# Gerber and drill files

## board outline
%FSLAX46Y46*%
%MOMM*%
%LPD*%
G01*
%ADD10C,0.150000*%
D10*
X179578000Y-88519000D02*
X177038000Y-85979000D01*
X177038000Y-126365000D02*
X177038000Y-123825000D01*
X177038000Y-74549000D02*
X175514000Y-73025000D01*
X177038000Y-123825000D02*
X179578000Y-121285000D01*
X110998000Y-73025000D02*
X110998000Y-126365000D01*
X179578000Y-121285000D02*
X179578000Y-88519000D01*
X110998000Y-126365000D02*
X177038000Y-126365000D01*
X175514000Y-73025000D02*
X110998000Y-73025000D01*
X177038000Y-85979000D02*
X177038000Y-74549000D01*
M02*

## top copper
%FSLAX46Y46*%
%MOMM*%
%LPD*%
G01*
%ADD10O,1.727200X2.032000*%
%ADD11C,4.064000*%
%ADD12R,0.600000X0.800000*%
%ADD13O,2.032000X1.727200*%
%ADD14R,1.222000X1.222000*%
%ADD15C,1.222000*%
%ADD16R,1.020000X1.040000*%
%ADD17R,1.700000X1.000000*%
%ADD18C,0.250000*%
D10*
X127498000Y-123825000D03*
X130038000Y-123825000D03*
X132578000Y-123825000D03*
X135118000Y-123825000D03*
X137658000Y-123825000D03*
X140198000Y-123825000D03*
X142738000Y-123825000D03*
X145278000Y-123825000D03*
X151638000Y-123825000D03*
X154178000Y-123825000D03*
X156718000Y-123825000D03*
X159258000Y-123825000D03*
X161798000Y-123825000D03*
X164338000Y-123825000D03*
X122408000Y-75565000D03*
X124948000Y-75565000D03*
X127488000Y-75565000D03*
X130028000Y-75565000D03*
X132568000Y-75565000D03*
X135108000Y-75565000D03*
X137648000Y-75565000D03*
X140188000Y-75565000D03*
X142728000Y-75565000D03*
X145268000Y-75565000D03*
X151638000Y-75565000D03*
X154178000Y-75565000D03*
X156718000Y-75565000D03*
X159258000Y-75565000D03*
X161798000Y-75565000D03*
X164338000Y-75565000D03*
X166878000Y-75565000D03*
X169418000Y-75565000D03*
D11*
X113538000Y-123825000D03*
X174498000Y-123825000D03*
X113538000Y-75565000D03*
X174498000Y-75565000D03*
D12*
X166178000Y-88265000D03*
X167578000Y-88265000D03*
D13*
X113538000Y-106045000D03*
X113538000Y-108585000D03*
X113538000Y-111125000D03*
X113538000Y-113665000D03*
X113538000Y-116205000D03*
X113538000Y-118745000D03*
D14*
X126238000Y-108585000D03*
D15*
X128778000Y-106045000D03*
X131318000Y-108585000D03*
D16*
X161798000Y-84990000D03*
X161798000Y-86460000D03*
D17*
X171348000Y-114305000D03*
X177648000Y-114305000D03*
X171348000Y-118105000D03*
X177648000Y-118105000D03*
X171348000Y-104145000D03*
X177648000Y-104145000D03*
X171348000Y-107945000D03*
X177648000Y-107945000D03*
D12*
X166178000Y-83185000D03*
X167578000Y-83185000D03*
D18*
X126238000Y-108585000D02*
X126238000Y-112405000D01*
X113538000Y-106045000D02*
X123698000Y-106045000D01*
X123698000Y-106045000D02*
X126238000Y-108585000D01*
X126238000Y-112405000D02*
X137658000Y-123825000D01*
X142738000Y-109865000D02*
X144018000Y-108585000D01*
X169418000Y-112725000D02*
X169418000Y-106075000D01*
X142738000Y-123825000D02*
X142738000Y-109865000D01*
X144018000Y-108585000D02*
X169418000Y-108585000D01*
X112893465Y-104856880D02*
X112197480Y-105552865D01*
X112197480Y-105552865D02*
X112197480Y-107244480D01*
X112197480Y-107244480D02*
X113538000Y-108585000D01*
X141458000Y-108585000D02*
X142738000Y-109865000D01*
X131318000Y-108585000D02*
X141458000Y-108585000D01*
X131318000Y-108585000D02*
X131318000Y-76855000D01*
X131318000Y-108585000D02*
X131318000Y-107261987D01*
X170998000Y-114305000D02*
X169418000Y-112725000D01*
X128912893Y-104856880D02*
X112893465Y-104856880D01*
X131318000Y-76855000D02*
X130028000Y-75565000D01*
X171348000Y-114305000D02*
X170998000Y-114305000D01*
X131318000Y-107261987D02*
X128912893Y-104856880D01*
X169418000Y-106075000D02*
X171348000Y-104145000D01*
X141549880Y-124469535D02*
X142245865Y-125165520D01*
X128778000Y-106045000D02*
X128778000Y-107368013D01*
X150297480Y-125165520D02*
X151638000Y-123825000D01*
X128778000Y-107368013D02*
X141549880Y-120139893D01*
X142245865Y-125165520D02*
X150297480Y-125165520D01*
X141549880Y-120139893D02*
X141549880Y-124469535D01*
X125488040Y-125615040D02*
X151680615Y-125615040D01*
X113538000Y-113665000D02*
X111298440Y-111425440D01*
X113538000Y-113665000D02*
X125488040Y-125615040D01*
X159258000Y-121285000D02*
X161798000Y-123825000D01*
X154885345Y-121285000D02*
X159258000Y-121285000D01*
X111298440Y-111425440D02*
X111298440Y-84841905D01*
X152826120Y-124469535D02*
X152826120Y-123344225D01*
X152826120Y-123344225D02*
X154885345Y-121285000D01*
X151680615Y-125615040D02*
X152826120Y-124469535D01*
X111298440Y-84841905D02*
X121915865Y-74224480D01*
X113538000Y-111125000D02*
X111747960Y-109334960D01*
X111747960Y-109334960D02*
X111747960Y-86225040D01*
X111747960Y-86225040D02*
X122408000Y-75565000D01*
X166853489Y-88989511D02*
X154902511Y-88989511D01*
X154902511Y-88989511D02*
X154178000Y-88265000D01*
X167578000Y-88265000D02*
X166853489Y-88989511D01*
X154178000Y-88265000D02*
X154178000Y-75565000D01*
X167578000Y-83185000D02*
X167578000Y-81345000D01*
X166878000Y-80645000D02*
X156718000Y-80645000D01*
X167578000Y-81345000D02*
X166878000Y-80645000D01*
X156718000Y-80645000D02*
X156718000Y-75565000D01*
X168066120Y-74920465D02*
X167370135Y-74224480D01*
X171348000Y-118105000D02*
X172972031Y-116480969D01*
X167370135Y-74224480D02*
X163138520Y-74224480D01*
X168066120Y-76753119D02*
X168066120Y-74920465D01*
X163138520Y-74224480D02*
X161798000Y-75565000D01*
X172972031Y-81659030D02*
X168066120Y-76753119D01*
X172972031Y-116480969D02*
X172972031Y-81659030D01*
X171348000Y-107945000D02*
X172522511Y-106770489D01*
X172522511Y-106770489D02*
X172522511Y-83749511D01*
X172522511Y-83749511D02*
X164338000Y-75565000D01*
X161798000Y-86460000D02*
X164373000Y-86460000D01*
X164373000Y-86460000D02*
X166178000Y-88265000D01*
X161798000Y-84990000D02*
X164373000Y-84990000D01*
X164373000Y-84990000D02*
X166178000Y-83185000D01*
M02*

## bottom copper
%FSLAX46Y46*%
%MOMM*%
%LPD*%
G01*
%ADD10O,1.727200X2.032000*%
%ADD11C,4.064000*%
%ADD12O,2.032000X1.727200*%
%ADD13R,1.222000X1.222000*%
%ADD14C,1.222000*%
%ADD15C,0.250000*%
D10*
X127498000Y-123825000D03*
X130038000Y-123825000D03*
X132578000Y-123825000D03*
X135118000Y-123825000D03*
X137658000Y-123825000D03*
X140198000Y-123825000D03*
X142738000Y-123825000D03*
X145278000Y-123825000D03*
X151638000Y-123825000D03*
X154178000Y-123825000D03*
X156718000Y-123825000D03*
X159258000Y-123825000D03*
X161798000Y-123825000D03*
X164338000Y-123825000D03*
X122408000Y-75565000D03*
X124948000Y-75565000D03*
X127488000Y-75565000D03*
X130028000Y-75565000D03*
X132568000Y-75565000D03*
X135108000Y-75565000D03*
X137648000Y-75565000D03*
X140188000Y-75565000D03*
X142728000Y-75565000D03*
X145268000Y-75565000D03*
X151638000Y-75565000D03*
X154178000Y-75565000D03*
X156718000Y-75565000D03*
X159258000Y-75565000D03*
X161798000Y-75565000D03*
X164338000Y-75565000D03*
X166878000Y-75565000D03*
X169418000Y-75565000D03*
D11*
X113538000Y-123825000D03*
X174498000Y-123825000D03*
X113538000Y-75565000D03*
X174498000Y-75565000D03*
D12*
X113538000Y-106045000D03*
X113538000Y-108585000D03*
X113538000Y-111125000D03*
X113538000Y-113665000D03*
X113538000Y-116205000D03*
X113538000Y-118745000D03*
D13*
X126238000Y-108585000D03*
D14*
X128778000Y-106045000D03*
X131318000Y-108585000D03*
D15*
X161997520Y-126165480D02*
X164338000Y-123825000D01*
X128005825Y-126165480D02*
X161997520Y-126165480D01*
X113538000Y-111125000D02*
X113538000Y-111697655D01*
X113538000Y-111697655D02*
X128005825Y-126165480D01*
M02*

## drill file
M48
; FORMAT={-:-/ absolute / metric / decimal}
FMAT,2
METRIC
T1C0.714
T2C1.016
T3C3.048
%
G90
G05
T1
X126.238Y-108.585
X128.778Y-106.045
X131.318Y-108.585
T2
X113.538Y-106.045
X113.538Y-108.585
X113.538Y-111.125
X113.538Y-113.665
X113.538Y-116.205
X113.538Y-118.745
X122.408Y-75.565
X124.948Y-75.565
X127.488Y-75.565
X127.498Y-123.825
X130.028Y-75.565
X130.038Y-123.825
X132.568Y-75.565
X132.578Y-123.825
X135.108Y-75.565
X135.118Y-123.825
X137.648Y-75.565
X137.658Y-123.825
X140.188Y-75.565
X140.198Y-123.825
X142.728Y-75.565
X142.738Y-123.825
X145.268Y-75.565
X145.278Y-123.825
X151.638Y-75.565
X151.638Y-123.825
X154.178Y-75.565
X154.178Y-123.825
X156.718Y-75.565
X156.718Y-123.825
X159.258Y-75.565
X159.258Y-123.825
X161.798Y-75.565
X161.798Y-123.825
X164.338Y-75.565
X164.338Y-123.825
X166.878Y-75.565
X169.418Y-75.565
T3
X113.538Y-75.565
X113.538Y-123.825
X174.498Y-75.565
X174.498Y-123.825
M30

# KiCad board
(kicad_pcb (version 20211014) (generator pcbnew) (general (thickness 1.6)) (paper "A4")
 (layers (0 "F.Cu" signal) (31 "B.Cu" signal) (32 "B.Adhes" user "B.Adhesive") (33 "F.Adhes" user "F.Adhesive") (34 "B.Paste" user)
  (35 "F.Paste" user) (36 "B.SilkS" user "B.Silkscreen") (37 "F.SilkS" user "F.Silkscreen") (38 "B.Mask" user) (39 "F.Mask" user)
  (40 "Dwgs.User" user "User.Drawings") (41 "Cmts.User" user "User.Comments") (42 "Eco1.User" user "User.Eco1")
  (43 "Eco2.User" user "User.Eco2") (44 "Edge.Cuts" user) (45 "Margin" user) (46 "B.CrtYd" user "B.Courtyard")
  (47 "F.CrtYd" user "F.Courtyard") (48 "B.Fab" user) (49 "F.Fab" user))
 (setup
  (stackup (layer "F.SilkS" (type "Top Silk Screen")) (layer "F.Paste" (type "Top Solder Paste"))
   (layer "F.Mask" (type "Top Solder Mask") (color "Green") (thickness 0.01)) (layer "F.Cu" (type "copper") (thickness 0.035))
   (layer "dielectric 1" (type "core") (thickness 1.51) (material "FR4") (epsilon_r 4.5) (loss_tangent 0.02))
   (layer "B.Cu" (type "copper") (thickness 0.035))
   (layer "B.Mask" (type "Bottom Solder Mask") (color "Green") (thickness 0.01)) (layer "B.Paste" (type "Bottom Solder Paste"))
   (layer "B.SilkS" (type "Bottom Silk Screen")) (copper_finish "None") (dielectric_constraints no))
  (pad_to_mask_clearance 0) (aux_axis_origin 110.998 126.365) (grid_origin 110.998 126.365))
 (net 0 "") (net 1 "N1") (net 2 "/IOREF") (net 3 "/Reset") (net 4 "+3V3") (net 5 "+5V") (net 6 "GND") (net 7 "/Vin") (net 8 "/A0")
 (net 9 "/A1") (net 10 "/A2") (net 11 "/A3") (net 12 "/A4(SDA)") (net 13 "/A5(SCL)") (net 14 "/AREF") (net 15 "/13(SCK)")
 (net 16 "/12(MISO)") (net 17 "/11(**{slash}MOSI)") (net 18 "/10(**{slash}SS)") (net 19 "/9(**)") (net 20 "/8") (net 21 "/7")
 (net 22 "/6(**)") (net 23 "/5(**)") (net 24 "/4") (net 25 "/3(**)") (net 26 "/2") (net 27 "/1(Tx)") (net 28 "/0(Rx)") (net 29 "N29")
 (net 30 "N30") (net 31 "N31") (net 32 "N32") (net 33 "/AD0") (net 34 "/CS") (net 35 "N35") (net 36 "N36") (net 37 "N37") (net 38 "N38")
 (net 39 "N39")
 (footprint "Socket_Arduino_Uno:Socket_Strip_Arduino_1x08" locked (layer "F.Cu") (at 127.498 123.825)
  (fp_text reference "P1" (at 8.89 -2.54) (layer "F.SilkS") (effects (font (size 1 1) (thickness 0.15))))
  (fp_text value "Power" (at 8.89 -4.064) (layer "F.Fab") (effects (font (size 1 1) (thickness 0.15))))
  (pad "1" thru_hole oval locked (at 0 0) (size 1.7272 2.032) (drill 1.016) (layers *.Cu *.Mask "F.SilkS") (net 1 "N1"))
  (pad "2" thru_hole oval locked (at 2.54 0) (size 1.7272 2.032) (drill 1.016) (layers *.Cu *.Mask "F.SilkS") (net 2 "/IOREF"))
  (pad "3" thru_hole oval locked (at 5.08 0) (size 1.7272 2.032) (drill 1.016) (layers *.Cu *.Mask "F.SilkS") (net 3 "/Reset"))
  (pad "4" thru_hole oval locked (at 7.62 0) (size 1.7272 2.032) (drill 1.016) (layers *.Cu *.Mask "F.SilkS") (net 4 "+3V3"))
  (pad "5" thru_hole oval locked (at 10.16 0) (size 1.7272 2.032) (drill 1.016) (layers *.Cu *.Mask "F.SilkS") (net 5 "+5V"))
  (pad "6" thru_hole oval locked (at 12.7 0) (size 1.7272 2.032) (drill 1.016) (layers *.Cu *.Mask "F.SilkS") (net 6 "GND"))
  (pad "7" thru_hole oval locked (at 15.24 0) (size 1.7272 2.032) (drill 1.016) (layers *.Cu *.Mask "F.SilkS") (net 6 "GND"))
  (pad "8" thru_hole oval locked (at 17.78 0) (size 1.7272 2.032) (drill 1.016) (layers *.Cu *.Mask "F.SilkS") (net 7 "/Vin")))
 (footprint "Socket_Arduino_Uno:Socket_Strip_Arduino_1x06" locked (layer "F.Cu") (at 151.638 123.825)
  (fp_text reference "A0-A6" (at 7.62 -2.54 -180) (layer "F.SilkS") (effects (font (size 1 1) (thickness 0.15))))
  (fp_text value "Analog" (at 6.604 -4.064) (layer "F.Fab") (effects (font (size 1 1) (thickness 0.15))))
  (pad "1" thru_hole oval locked (at 0 0) (size 1.7272 2.032) (drill 1.016) (layers *.Cu *.Mask "F.SilkS") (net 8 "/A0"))
  (pad "2" thru_hole oval locked (at 2.54 0) (size 1.7272 2.032) (drill 1.016) (layers *.Cu *.Mask "F.SilkS") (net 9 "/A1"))
  (pad "3" thru_hole oval locked (at 5.08 0) (size 1.7272 2.032) (drill 1.016) (layers *.Cu *.Mask "F.SilkS") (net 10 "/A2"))
  (pad "4" thru_hole oval locked (at 7.62 0) (size 1.7272 2.032) (drill 1.016) (layers *.Cu *.Mask "F.SilkS") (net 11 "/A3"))
  (pad "5" thru_hole oval locked (at 10.16 0) (size 1.7272 2.032) (drill 1.016) (layers *.Cu *.Mask "F.SilkS") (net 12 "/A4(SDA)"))
  (pad "6" thru_hole oval locked (at 12.7 0) (size 1.7272 2.032) (drill 1.016) (layers *.Cu *.Mask "F.SilkS") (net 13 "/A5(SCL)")))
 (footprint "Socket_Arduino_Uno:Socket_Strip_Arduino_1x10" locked (layer "F.Cu") (at 122.408 75.565)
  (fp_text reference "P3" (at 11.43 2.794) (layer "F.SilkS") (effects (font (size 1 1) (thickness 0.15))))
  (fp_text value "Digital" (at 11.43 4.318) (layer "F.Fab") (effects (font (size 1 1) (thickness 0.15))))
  (pad "1" thru_hole oval locked (at 0 0) (size 1.7272 2.032) (drill 1.016) (layers *.Cu *.Mask "F.SilkS") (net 13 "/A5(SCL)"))
  (pad "2" thru_hole oval locked (at 2.54 0) (size 1.7272 2.032) (drill 1.016) (layers *.Cu *.Mask "F.SilkS") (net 12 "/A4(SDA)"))
  (pad "3" thru_hole oval locked (at 5.08 0) (size 1.7272 2.032) (drill 1.016) (layers *.Cu *.Mask "F.SilkS") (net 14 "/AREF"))
  (pad "4" thru_hole oval locked (at 7.62 0) (size 1.7272 2.032) (drill 1.016) (layers *.Cu *.Mask "F.SilkS") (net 6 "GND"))
  (pad "5" thru_hole oval locked (at 10.16 0) (size 1.7272 2.032) (drill 1.016) (layers *.Cu *.Mask "F.SilkS") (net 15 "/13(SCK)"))
  (pad "6" thru_hole oval locked (at 12.7 0) (size 1.7272 2.032) (drill 1.016) (layers *.Cu *.Mask "F.SilkS") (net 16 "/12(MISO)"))
  (pad "7" thru_hole oval locked (at 15.24 0) (size 1.7272 2.032) (drill 1.016) (layers *.Cu *.Mask "F.SilkS") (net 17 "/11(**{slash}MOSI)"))
  (pad "8" thru_hole oval locked (at 17.78 0) (size 1.7272 2.032) (drill 1.016) (layers *.Cu *.Mask "F.SilkS") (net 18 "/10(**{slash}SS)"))
  (pad "9" thru_hole oval locked (at 20.32 0) (size 1.7272 2.032) (drill 1.016) (layers *.Cu *.Mask "F.SilkS") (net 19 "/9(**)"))
  (pad "10" thru_hole oval locked (at 22.86 0) (size 1.7272 2.032) (drill 1.016) (layers *.Cu *.Mask "F.SilkS") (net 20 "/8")))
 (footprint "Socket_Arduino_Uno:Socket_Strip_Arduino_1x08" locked (layer "F.Cu") (at 151.638 75.565)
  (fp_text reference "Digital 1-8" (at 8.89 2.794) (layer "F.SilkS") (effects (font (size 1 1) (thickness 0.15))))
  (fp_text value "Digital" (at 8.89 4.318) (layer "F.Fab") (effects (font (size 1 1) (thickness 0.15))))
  (pad "1" thru_hole oval locked (at 0 0) (size 1.7272 2.032) (drill 1.016) (layers *.Cu *.Mask "F.SilkS") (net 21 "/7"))
  (pad "2" thru_hole oval locked (at 2.54 0) (size 1.7272 2.032) (drill 1.016) (layers *.Cu *.Mask "F.SilkS") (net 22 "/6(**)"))
  (pad "3" thru_hole oval locked (at 5.08 0) (size 1.7272 2.032) (drill 1.016) (layers *.Cu *.Mask "F.SilkS") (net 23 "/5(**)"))
  (pad "4" thru_hole oval locked (at 7.62 0) (size 1.7272 2.032) (drill 1.016) (layers *.Cu *.Mask "F.SilkS") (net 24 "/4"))
  (pad "5" thru_hole oval locked (at 10.16 0) (size 1.7272 2.032) (drill 1.016) (layers *.Cu *.Mask "F.SilkS") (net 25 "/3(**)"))
  (pad "6" thru_hole oval locked (at 12.7 0) (size 1.7272 2.032) (drill 1.016) (layers *.Cu *.Mask "F.SilkS") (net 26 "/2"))
  (pad "7" thru_hole oval locked (at 15.24 0) (size 1.7272 2.032) (drill 1.016) (layers *.Cu *.Mask "F.SilkS") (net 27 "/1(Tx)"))
  (pad "8" thru_hole oval locked (at 17.78 0) (size 1.7272 2.032) (drill 1.016) (layers *.Cu *.Mask "F.SilkS") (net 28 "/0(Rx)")))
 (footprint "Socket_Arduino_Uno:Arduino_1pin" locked (layer "F.Cu") (at 113.538 123.825)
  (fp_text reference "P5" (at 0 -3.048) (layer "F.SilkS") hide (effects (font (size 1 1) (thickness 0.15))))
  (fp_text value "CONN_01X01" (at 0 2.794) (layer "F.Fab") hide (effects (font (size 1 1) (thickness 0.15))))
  (pad "1" thru_hole circle locked (at 0 0) (size 4.064 4.064) (drill 3.048) (layers *.Cu *.Mask "F.SilkS") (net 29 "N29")))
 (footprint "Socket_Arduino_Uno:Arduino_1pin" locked (layer "F.Cu") (at 174.498 123.825)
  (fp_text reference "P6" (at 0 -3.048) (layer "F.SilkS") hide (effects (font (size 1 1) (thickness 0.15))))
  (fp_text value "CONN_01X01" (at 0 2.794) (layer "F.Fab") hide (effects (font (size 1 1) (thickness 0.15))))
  (pad "1" thru_hole circle locked (at 0 0) (size 4.064 4.064) (drill 3.048) (layers *.Cu *.Mask "F.SilkS") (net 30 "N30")))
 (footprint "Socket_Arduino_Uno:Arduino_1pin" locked (layer "F.Cu") (at 113.538 75.565)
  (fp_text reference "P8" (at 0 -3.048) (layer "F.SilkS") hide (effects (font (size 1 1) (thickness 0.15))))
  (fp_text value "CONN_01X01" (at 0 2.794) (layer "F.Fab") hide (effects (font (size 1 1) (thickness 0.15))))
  (pad "1" thru_hole circle locked (at 0 0) (size 4.064 4.064) (drill 3.048) (layers *.Cu *.Mask "F.SilkS") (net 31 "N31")))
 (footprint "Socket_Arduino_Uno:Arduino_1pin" (layer "F.Cu") (at 174.498 75.565)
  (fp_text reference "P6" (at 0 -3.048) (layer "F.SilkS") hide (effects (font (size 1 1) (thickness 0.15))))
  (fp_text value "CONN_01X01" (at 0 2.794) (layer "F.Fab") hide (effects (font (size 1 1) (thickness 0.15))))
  (pad "1" thru_hole circle locked (at 0 0) (size 4.064 4.064) (drill 3.048) (layers *.Cu *.Mask "F.SilkS")))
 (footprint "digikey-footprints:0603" (layer "F.Cu") (at 166.878 88.265)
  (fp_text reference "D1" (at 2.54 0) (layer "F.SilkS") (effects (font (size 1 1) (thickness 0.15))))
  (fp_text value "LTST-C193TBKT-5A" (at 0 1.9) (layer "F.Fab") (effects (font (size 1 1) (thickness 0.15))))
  (pad "1" smd rect locked (at -0.7 0) (size 0.6 0.8) (layers "F.Cu" "F.Paste" "F.Mask") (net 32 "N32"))
  (pad "2" smd rect locked (at 0.7 0) (size 0.6 0.8) (layers "F.Cu" "F.Paste" "F.Mask") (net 22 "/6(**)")))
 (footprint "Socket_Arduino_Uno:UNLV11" (layer "F.Cu") (at 121.158 83.185)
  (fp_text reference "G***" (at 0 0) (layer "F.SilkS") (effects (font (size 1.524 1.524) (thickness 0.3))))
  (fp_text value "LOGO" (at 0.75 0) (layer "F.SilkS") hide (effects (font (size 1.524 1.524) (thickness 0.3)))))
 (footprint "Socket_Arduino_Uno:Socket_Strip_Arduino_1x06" (layer "F.Cu") (at 113.538 106.045 -90)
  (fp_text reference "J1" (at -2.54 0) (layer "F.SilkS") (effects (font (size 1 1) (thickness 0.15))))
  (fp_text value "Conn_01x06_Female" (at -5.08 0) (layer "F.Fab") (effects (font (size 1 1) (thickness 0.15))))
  (pad "1" thru_hole oval locked (at 0 0 270) (size 1.7272 2.032) (drill 1.016) (layers *.Cu *.Mask "F.SilkS") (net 5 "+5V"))
  (pad "2" thru_hole oval locked (at 2.54 0 270) (size 1.7272 2.032) (drill 1.016) (layers *.Cu *.Mask "F.SilkS") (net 6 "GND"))
  (pad "3" thru_hole oval locked (at 5.08 0 270) (size 1.7272 2.032) (drill 1.016) (layers *.Cu *.Mask "F.SilkS") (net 13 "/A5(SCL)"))
  (pad "4" thru_hole oval locked (at 7.62 0 270) (size 1.7272 2.032) (drill 1.016) (layers *.Cu *.Mask "F.SilkS") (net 12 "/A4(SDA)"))
  (pad "5" thru_hole oval locked (at 10.16 0 270) (size 1.7272 2.032) (drill 1.016) (layers *.Cu *.Mask "F.SilkS") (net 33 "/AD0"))
  (pad "6" thru_hole oval locked (at 12.7 0 270) (size 1.7272 2.032) (drill 1.016) (layers *.Cu *.Mask "F.SilkS") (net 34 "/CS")))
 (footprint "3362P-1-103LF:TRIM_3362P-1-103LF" (layer "F.Cu") (at 128.778 108.585)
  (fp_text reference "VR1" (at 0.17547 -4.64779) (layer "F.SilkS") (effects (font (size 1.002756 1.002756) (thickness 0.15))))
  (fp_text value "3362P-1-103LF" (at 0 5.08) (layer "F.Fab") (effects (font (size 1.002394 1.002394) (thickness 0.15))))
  (pad "1" thru_hole rect locked (at -2.54 0) (size 1.222 1.222) (drill 0.714) (layers *.Cu *.Mask) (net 5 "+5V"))
  (pad "2" thru_hole circle locked (at 0 -2.54) (size 1.222 1.222) (drill 0.714) (layers *.Cu *.Mask) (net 8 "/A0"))
  (pad "3" thru_hole circle locked (at 2.54 0) (size 1.222 1.222) (drill 0.714) (layers *.Cu *.Mask) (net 6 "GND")))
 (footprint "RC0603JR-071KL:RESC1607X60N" (layer "F.Cu") (at 161.798 85.725 -90)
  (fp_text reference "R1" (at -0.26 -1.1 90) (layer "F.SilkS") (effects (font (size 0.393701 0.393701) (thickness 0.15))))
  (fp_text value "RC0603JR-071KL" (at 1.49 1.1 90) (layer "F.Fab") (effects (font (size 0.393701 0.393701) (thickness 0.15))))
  (pad "1" smd rect locked (at -0.735 0 270) (size 1.04 1.02) (layers "F.Cu" "F.Paste" "F.Mask") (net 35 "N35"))
  (pad "2" smd rect locked (at 0.735 0 270) (size 1.04 1.02) (layers "F.Cu" "F.Paste" "F.Mask") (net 32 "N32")))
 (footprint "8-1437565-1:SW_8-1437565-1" (layer "F.Cu") (at 174.498 116.205)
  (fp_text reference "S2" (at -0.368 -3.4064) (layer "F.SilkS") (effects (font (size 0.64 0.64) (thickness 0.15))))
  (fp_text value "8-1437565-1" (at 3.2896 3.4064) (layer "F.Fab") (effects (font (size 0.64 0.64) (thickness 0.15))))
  (pad "1" smd rect locked (at -3.15 -1.9) (size 1.7 1) (layers "F.Cu" "F.Paste" "F.Mask") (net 6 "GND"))
  (pad "2" smd rect locked (at 3.15 -1.9) (size 1.7 1) (layers "F.Cu" "F.Paste" "F.Mask") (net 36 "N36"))
  (pad "3" smd rect locked (at -3.15 1.9) (size 1.7 1) (layers "F.Cu" "F.Paste" "F.Mask") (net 25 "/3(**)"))
  (pad "4" smd rect locked (at 3.15 1.9) (size 1.7 1) (layers "F.Cu" "F.Paste" "F.Mask") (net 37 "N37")))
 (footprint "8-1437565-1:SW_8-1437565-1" (layer "F.Cu") (at 174.498 106.045)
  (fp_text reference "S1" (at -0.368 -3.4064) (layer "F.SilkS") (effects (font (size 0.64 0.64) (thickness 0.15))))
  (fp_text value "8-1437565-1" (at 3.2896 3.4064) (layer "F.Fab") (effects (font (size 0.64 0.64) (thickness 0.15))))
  (pad "1" smd rect locked (at -3.15 -1.9) (size 1.7 1) (layers "F.Cu" "F.Paste" "F.Mask") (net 6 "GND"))
  (pad "2" smd rect locked (at 3.15 -1.9) (size 1.7 1) (layers "F.Cu" "F.Paste" "F.Mask") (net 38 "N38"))
  (pad "3" smd rect locked (at -3.15 1.9) (size 1.7 1) (layers "F.Cu" "F.Paste" "F.Mask") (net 26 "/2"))
  (pad "4" smd rect locked (at 3.15 1.9) (size 1.7 1) (layers "F.Cu" "F.Paste" "F.Mask") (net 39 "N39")))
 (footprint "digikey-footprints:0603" (layer "F.Cu") (at 166.878 83.185)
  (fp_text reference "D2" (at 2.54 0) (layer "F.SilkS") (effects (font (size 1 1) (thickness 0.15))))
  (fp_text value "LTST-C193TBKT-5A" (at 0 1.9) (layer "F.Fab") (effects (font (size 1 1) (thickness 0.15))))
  (pad "1" smd rect locked (at -0.7 0) (size 0.6 0.8) (layers "F.Cu" "F.Paste" "F.Mask") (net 35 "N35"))
  (pad "2" smd rect locked (at 0.7 0) (size 0.6 0.8) (layers "F.Cu" "F.Paste" "F.Mask") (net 23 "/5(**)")))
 (gr_line (start 179.578 88.519) (end 177.038 85.979) (layer "Edge.Cuts") (width 0.15))
 (gr_line (start 177.038 126.365) (end 177.038 123.825) (layer "Edge.Cuts") (width 0.15))
 (gr_line (start 177.038 74.549) (end 175.514 73.025) (layer "Edge.Cuts") (width 0.15))
 (gr_line (start 177.038 123.825) (end 179.578 121.285) (layer "Edge.Cuts") (width 0.15))
 (gr_line (start 110.998 73.025) (end 110.998 126.365) (layer "Edge.Cuts") (width 0.15))
 (gr_line (start 179.578 121.285) (end 179.578 88.519) (layer "Edge.Cuts") (width 0.15))
 (gr_line (start 110.998 126.365) (end 177.038 126.365) (layer "Edge.Cuts") (width 0.15))
 (gr_line (start 175.514 73.025) (end 110.998 73.025) (layer "Edge.Cuts") (width 0.15))
 (gr_line (start 177.038 85.979) (end 177.038 74.549) (layer "Edge.Cuts") (width 0.15))
 (segment (start 126.238 108.585) (end 126.238 112.405) (width 0.25) (layer "F.Cu") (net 5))
 (segment (start 113.538 106.045) (end 123.698 106.045) (width 0.25) (layer "F.Cu") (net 5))
 (segment (start 123.698 106.045) (end 126.238 108.585) (width 0.25) (layer "F.Cu") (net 5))
 (segment (start 126.238 112.405) (end 137.658 123.825) (width 0.25) (layer "F.Cu") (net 5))
 (segment (start 142.738 109.865) (end 144.018 108.585) (width 0.25) (layer "F.Cu") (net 6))
 (segment (start 169.418 112.725) (end 169.418 106.075) (width 0.25) (layer "F.Cu") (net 6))
 (segment (start 142.738 123.825) (end 142.738 109.865) (width 0.25) (layer "F.Cu") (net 6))
 (segment (start 144.018 108.585) (end 169.418 108.585) (width 0.25) (layer "F.Cu") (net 6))
 (segment (start 112.893465 104.85688) (end 112.19748 105.552865) (width 0.25) (layer "F.Cu") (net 6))
 (segment (start 112.19748 105.552865) (end 112.19748 107.24448) (width 0.25) (layer "F.Cu") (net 6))
 (segment (start 112.19748 107.24448) (end 113.538 108.585) (width 0.25) (layer "F.Cu") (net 6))
 (segment (start 141.458 108.585) (end 142.738 109.865) (width 0.25) (layer "F.Cu") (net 6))
 (segment (start 131.318 108.585) (end 141.458 108.585) (width 0.25) (layer "F.Cu") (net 6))
 (segment (start 131.318 108.585) (end 131.318 76.855) (width 0.25) (layer "F.Cu") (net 6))
 (segment (start 131.318 108.585) (end 131.318 107.261987) (width 0.25) (layer "F.Cu") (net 6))
 (segment (start 170.998 114.305) (end 169.418 112.725) (width 0.25) (layer "F.Cu") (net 6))
 (segment (start 128.912893 104.85688) (end 112.893465 104.85688) (width 0.25) (layer "F.Cu") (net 6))
 (segment (start 131.318 76.855) (end 130.028 75.565) (width 0.25) (layer "F.Cu") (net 6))
 (segment (start 171.348 114.305) (end 170.998 114.305) (width 0.25) (layer "F.Cu") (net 6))
 (segment (start 131.318 107.261987) (end 128.912893 104.85688) (width 0.25) (layer "F.Cu") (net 6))
 (segment (start 169.418 106.075) (end 171.348 104.145) (width 0.25) (layer "F.Cu") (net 6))
 (segment (start 141.54988 124.469535) (end 142.245865 125.16552) (width 0.25) (layer "F.Cu") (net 8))
 (segment (start 128.778 106.045) (end 128.778 107.368013) (width 0.25) (layer "F.Cu") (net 8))
 (segment (start 150.29748 125.16552) (end 151.638 123.825) (width 0.25) (layer "F.Cu") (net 8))
 (segment (start 128.778 107.368013) (end 141.54988 120.139893) (width 0.25) (layer "F.Cu") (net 8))
 (segment (start 142.245865 125.16552) (end 150.29748 125.16552) (width 0.25) (layer "F.Cu") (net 8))
 (segment (start 141.54988 120.139893) (end 141.54988 124.469535) (width 0.25) (layer "F.Cu") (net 8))
 (segment (start 125.48804 125.61504) (end 151.680615 125.61504) (width 0.25) (layer "F.Cu") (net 12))
 (segment (start 113.538 113.665) (end 111.29844 111.42544) (width 0.25) (layer "F.Cu") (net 12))
 (segment (start 113.538 113.665) (end 125.48804 125.61504) (width 0.25) (layer "F.Cu") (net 12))
 (segment (start 159.258 121.285) (end 161.798 123.825) (width 0.25) (layer "F.Cu") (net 12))
 (segment (start 154.885345 121.285) (end 159.258 121.285) (width 0.25) (layer "F.Cu") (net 12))
 (segment (start 111.29844 111.42544) (end 111.29844 84.841905) (width 0.25) (layer "F.Cu") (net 12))
 (segment (start 152.82612 124.469535) (end 152.82612 123.344225) (width 0.25) (layer "F.Cu") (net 12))
 (segment (start 152.82612 123.344225) (end 154.885345 121.285) (width 0.25) (layer "F.Cu") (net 12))
 (segment (start 151.680615 125.61504) (end 152.82612 124.469535) (width 0.25) (layer "F.Cu") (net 12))
 (segment (start 111.29844 84.841905) (end 121.915865 74.22448) (width 0.25) (layer "F.Cu") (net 12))
 (segment (start 113.538 111.125) (end 111.74796 109.33496) (width 0.25) (layer "F.Cu") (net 13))
 (segment (start 111.74796 109.33496) (end 111.74796 86.22504) (width 0.25) (layer "F.Cu") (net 13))
 (segment (start 111.74796 86.22504) (end 122.408 75.565) (width 0.25) (layer "F.Cu") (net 13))
 (segment (start 161.99752 126.16548) (end 164.338 123.825) (width 0.25) (layer "B.Cu") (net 13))
 (segment (start 128.005825 126.16548) (end 161.99752 126.16548) (width 0.25) (layer "B.Cu") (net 13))
 (segment (start 113.538 111.125) (end 113.538 111.697655) (width 0.25) (layer "B.Cu") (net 13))
 (segment (start 113.538 111.697655) (end 128.005825 126.16548) (width 0.25) (layer "B.Cu") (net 13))
 (segment (start 166.853489 88.989511) (end 154.902511 88.989511) (width 0.25) (layer "F.Cu") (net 22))
 (segment (start 154.902511 88.989511) (end 154.178 88.265) (width 0.25) (layer "F.Cu") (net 22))
 (segment (start 167.578 88.265) (end 166.853489 88.989511) (width 0.25) (layer "F.Cu") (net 22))
 (segment (start 154.178 88.265) (end 154.178 75.565) (width 0.25) (layer "F.Cu") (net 22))
 (segment (start 167.578 83.185) (end 167.578 81.345) (width 0.25) (layer "F.Cu") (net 23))
 (segment (start 166.878 80.645) (end 156.718 80.645) (width 0.25) (layer "F.Cu") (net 23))
 (segment (start 167.578 81.345) (end 166.878 80.645) (width 0.25) (layer "F.Cu") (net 23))
 (segment (start 156.718 80.645) (end 156.718 75.565) (width 0.25) (layer "F.Cu") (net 23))
 (segment (start 168.06612 74.920465) (end 167.370135 74.22448) (width 0.25) (layer "F.Cu") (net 25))
 (segment (start 171.348 118.105) (end 172.972031 116.480969) (width 0.25) (layer "F.Cu") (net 25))
 (segment (start 167.370135 74.22448) (end 163.13852 74.22448) (width 0.25) (layer "F.Cu") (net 25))
 (segment (start 168.06612 76.753119) (end 168.06612 74.920465) (width 0.25) (layer "F.Cu") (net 25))
 (segment (start 163.13852 74.22448) (end 161.798 75.565) (width 0.25) (layer "F.Cu") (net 25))
 (segment (start 172.972031 81.65903) (end 168.06612 76.753119) (width 0.25) (layer "F.Cu") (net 25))
 (segment (start 172.972031 116.480969) (end 172.972031 81.65903) (width 0.25) (layer "F.Cu") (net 25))
 (segment (start 171.348 107.945) (end 172.522511 106.770489) (width 0.25) (layer "F.Cu") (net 26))
 (segment (start 172.522511 106.770489) (end 172.522511 83.749511) (width 0.25) (layer "F.Cu") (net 26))
 (segment (start 172.522511 83.749511) (end 164.338 75.565) (width 0.25) (layer "F.Cu") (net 26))
 (segment (start 161.798 86.46) (end 164.373 86.46) (width 0.25) (layer "F.Cu") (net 32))
 (segment (start 164.373 86.46) (end 166.178 88.265) (width 0.25) (layer "F.Cu") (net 32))
 (segment (start 161.798 84.99) (end 164.373 84.99) (width 0.25) (layer "F.Cu") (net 35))
 (segment (start 164.373 84.99) (end 166.178 83.185) (width 0.25) (layer "F.Cu") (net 35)))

